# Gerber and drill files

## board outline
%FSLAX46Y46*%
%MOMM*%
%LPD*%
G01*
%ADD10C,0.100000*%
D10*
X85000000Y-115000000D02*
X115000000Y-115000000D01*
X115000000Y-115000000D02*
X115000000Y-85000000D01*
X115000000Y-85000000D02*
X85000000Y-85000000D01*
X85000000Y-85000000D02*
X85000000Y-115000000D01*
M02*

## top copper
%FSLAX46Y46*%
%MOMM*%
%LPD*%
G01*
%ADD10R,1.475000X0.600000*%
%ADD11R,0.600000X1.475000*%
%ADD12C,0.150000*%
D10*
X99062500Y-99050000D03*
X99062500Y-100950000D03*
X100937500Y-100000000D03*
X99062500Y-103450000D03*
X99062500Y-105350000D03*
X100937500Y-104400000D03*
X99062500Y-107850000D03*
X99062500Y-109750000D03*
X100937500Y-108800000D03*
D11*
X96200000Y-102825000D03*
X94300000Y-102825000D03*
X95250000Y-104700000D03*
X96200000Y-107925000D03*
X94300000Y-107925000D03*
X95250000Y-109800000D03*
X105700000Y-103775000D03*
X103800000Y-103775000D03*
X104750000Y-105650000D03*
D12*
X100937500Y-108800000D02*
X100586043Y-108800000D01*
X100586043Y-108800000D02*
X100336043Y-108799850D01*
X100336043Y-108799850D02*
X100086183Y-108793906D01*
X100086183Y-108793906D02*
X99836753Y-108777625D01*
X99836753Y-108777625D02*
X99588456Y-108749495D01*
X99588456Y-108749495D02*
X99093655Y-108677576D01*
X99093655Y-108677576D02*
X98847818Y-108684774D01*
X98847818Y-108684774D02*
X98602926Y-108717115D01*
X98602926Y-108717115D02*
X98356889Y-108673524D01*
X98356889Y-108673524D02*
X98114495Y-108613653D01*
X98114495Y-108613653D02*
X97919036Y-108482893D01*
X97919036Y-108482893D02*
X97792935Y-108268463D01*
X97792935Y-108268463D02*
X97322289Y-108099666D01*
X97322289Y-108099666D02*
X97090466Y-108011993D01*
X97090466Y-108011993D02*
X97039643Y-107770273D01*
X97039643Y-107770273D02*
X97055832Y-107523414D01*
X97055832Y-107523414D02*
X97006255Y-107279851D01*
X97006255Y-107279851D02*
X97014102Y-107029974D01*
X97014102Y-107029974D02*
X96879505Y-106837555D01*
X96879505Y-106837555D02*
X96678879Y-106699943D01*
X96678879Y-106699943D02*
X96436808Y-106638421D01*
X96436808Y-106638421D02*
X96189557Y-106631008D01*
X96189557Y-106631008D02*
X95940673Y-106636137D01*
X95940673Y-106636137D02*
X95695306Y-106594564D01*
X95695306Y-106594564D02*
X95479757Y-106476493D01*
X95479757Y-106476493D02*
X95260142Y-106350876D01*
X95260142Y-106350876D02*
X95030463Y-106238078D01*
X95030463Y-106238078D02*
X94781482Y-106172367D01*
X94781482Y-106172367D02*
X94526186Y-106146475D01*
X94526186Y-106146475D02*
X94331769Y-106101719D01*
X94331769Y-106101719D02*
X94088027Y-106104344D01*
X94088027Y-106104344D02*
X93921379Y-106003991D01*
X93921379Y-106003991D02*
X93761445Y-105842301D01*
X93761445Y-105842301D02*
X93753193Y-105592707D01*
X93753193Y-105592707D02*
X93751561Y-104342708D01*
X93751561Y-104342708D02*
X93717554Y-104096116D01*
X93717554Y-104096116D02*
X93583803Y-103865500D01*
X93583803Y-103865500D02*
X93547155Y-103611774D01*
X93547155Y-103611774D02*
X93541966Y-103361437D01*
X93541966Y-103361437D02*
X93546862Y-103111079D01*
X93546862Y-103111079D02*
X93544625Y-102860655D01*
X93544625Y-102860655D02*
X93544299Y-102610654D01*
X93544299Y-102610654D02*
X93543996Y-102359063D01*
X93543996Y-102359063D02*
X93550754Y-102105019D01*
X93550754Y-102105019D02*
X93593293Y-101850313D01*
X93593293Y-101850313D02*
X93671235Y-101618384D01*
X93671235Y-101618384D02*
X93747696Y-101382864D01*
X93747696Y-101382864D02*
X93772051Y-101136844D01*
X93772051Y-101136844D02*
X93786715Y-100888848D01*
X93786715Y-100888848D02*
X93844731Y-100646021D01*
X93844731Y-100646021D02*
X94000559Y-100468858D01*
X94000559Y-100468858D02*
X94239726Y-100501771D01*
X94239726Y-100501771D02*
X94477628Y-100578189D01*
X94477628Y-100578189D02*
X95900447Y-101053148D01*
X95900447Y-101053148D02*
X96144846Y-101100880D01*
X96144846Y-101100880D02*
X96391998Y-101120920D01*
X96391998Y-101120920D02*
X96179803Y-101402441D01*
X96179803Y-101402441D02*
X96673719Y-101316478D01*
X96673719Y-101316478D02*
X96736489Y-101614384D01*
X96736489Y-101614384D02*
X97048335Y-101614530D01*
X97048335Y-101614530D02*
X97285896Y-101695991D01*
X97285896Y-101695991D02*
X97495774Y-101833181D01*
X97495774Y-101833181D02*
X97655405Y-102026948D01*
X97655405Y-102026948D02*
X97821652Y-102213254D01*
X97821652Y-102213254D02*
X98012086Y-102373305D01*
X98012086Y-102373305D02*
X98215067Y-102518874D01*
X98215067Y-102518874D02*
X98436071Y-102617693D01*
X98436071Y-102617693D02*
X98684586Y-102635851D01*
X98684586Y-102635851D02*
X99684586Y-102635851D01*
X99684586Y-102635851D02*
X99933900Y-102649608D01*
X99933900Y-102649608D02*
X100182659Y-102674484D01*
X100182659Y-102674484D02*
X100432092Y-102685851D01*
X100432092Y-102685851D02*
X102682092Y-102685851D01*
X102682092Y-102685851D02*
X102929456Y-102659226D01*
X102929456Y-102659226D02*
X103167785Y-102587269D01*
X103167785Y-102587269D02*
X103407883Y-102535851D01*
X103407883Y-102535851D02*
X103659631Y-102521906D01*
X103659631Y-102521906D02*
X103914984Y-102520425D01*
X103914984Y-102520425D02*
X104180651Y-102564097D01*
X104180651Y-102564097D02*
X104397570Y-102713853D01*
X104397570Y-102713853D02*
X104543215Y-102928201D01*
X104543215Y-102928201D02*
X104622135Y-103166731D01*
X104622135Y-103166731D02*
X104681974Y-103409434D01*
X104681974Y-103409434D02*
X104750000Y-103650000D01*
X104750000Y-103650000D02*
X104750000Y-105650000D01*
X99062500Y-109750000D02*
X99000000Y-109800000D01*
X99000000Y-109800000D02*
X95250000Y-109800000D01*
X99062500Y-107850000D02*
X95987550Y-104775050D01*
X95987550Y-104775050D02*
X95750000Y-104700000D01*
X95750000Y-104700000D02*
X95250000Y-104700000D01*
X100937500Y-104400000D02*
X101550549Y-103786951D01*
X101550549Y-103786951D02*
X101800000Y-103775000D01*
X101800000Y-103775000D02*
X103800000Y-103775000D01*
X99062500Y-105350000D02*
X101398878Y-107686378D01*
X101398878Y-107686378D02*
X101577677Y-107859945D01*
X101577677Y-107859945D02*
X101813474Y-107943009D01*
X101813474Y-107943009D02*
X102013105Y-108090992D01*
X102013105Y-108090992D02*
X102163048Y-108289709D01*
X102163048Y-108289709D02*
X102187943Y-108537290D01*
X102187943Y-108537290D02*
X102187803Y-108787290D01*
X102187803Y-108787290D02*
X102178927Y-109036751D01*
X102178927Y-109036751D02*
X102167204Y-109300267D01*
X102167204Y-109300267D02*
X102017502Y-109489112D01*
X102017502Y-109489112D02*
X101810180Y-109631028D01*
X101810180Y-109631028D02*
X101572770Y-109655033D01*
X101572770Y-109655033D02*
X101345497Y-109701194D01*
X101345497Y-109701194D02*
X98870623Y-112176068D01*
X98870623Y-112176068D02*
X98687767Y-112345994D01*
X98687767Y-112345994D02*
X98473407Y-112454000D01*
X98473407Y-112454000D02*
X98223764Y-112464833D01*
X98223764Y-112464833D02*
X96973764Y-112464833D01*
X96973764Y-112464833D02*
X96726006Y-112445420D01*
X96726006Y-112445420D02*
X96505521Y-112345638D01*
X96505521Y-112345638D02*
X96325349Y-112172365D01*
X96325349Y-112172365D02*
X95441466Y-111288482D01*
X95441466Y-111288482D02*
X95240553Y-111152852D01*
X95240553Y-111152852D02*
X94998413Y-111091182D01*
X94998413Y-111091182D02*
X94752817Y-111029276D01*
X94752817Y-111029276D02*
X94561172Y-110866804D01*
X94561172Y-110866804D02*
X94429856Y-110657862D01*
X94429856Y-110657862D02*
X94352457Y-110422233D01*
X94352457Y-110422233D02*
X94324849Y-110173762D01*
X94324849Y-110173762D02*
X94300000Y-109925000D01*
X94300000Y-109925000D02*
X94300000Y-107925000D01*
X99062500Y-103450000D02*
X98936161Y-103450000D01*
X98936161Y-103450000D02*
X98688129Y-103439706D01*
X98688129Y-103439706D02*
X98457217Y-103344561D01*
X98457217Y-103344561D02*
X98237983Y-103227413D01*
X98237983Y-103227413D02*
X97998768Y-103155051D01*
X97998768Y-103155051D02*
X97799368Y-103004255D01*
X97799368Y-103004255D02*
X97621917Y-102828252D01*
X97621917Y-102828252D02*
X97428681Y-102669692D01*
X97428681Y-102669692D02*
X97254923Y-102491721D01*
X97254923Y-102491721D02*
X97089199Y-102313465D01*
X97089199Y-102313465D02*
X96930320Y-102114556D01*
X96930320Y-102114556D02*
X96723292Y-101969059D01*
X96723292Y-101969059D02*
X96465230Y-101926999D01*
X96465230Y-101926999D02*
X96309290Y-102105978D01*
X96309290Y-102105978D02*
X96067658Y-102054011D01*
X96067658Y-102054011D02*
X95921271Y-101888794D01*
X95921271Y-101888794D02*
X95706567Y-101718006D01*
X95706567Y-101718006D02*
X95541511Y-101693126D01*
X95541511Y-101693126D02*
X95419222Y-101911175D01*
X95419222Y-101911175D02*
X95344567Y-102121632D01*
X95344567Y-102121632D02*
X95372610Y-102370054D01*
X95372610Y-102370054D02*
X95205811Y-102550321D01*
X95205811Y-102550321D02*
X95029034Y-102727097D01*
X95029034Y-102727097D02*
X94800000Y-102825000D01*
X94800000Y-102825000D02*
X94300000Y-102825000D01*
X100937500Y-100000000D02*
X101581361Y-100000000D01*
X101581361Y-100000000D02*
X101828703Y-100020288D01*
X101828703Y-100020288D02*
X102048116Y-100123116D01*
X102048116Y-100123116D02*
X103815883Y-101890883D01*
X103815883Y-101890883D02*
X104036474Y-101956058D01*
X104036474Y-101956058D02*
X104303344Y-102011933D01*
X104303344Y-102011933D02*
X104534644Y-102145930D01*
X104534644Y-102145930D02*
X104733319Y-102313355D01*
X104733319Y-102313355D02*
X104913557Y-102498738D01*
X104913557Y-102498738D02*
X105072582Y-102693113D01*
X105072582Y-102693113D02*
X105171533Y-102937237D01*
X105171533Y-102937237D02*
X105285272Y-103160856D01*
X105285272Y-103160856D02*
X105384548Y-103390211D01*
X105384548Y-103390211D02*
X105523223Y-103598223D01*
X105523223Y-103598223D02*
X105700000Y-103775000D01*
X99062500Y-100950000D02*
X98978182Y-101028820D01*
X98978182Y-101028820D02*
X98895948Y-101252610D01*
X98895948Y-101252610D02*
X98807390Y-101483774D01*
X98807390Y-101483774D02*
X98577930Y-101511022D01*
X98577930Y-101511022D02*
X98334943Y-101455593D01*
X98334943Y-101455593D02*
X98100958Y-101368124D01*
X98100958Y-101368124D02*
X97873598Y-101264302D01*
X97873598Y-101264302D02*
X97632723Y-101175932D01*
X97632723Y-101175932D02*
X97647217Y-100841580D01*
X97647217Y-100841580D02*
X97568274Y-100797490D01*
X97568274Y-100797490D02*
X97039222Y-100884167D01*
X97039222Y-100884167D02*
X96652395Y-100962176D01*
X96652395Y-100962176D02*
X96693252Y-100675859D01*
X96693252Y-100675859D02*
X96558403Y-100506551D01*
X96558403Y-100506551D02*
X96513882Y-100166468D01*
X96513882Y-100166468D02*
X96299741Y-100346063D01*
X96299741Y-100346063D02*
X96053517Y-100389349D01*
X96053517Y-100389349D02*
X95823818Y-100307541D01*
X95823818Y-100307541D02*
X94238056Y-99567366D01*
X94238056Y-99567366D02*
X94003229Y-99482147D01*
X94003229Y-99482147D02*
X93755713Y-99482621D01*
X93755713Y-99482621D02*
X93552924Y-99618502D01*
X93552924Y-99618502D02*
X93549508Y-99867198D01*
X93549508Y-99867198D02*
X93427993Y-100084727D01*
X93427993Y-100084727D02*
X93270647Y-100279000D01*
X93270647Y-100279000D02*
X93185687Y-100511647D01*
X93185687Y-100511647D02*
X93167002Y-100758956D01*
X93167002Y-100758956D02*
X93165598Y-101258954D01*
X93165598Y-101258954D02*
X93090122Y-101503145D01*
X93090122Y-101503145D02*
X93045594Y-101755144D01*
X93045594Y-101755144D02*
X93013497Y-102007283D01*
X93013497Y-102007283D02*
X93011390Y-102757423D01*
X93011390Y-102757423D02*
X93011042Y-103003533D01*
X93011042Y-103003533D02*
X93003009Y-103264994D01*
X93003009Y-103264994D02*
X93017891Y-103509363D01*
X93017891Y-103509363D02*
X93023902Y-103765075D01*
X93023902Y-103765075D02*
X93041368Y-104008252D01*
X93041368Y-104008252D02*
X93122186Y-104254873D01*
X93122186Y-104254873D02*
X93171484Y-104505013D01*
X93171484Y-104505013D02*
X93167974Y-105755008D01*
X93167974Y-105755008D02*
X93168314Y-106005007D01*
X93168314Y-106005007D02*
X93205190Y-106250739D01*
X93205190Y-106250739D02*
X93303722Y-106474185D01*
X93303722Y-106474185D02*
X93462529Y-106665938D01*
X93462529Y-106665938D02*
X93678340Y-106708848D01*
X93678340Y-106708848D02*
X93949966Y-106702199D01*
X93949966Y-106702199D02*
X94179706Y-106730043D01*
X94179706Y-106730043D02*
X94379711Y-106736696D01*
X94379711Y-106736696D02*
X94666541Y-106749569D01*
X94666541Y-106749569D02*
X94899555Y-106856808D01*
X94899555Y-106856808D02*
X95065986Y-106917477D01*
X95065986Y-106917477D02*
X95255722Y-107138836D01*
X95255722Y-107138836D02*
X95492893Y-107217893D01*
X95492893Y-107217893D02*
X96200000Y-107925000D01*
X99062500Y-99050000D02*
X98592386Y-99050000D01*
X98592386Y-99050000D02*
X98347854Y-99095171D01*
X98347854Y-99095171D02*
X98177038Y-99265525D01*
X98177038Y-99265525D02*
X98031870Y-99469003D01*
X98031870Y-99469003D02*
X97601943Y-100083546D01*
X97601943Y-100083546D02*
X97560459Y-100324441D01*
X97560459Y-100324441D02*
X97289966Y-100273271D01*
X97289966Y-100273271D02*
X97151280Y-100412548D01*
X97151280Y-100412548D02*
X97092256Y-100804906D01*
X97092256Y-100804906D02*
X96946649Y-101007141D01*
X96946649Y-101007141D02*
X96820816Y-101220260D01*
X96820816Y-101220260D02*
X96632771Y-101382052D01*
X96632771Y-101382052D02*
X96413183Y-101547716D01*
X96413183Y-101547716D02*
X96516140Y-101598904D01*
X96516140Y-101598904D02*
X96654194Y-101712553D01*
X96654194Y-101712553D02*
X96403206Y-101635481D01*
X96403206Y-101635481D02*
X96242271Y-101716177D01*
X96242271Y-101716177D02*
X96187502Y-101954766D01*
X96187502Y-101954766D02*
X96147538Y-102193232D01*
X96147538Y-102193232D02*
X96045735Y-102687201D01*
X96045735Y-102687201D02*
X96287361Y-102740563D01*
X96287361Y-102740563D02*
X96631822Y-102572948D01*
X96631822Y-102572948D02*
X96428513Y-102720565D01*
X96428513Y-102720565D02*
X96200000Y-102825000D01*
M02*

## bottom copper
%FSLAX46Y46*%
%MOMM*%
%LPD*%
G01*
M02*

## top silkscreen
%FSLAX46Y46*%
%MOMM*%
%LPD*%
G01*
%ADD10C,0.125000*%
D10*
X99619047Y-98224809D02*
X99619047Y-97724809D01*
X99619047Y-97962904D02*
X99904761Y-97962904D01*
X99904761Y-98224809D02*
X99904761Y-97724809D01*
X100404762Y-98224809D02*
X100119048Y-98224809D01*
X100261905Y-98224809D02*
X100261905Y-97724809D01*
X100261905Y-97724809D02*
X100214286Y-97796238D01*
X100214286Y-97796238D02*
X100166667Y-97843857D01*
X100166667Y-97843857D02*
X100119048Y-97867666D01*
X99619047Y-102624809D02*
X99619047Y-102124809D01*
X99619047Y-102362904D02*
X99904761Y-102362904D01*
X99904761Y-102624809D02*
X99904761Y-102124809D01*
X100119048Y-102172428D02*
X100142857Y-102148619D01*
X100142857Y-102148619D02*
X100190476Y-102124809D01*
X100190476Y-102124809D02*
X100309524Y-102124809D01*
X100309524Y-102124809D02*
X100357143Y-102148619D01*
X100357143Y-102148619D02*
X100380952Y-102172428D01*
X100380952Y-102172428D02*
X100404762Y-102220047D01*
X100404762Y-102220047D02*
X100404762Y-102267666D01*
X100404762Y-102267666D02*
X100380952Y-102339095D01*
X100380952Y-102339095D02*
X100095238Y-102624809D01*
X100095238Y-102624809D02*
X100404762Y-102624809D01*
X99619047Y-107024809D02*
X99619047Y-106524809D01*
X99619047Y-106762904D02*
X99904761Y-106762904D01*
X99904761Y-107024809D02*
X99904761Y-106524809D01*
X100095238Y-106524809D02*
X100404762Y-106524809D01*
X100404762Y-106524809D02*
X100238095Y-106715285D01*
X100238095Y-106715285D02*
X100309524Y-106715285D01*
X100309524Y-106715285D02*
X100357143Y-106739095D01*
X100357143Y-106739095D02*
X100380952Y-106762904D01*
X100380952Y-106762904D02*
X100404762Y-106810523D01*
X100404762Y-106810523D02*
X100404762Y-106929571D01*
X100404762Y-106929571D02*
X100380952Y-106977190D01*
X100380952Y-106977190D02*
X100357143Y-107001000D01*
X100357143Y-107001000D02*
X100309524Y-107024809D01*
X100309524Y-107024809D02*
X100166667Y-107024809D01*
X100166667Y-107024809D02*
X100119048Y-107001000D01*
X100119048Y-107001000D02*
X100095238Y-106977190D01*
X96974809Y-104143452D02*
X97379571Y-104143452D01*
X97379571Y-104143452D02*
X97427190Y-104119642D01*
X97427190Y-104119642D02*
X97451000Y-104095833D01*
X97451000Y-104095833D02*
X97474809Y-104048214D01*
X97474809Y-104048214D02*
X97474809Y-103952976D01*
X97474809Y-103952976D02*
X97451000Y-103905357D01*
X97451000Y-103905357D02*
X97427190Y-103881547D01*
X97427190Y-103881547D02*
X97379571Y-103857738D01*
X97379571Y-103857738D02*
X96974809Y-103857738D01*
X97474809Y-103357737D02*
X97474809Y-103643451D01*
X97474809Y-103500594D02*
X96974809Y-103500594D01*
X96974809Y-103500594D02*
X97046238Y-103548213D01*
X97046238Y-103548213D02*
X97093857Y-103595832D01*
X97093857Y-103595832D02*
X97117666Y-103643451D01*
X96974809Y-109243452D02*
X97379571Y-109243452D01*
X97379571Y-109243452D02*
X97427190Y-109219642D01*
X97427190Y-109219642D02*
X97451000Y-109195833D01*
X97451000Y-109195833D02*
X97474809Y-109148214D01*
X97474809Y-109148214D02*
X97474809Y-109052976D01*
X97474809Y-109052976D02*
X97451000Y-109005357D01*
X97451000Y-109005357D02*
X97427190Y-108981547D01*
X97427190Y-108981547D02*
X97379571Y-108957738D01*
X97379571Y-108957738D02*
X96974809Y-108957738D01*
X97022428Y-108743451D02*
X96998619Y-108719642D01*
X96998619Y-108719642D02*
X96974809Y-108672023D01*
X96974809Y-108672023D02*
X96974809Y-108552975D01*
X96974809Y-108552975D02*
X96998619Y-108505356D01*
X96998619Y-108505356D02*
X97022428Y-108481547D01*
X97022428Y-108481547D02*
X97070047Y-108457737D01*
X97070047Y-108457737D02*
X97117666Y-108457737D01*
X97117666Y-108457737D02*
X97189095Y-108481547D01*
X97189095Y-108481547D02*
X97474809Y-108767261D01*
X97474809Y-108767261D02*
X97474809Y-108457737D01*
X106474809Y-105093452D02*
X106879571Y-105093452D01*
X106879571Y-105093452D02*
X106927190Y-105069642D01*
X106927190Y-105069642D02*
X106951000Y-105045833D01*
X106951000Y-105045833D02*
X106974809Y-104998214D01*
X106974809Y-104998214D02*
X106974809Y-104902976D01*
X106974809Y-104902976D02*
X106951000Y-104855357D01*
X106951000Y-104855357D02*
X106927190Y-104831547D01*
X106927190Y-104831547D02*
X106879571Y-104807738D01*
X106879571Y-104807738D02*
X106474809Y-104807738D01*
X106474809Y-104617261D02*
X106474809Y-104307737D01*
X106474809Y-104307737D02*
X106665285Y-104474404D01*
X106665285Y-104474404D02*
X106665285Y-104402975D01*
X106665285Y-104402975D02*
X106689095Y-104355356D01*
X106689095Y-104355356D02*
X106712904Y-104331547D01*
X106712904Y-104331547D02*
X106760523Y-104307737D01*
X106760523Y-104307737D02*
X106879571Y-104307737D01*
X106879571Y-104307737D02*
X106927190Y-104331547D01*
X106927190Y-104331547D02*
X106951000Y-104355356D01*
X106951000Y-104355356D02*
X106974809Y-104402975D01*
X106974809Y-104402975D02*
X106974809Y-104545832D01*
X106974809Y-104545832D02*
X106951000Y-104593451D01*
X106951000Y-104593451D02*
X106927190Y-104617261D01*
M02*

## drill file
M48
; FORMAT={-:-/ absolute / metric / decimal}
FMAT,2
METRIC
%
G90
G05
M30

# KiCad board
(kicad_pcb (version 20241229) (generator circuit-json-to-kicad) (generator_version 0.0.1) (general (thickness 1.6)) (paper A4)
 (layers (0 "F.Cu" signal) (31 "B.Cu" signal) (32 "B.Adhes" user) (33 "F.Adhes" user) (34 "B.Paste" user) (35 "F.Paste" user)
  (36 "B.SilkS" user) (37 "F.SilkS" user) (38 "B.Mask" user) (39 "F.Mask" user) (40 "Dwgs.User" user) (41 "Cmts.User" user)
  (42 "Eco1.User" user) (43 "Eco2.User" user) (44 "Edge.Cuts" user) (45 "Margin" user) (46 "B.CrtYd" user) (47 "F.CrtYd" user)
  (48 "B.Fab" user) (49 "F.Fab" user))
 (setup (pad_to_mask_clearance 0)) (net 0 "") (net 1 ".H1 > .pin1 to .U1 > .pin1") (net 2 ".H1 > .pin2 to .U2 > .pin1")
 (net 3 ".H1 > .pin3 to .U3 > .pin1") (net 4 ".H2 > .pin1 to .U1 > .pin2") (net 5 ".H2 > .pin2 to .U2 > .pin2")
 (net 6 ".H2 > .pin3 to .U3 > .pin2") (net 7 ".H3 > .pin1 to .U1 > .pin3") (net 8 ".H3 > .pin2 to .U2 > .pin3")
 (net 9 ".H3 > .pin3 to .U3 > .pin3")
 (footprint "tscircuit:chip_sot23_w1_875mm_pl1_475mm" (layer F.Cu) (at 100 100 0)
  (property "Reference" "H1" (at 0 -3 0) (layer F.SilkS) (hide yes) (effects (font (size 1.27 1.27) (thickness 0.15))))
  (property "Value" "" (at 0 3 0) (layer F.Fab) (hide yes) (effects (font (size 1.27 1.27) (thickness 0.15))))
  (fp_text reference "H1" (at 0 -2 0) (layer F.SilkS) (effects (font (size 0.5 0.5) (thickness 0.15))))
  (pad "1" smd rect (at -0.9375 -0.95 0) (size 1.475 0.6) (layers F.Cu F.Mask) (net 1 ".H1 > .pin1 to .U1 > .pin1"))
  (pad "2" smd rect (at -0.9375 0.95 0) (size 1.475 0.6) (layers F.Cu F.Mask) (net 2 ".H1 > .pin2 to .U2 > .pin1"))
  (pad "3" smd rect (at 0.9375 0 0) (size 1.475 0.6) (layers F.Cu F.Mask) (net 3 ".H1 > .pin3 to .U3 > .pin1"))
  (pad "" smd rect (at -0.9375 -0.95 0) (size 1.0325 0.42) (layers F.Paste))
  (pad "" smd rect (at -0.9375 0.95 0) (size 1.0325 0.42) (layers F.Paste))
  (pad "" smd rect (at 0.9375 0 0) (size 1.0325 0.42) (layers F.Paste)))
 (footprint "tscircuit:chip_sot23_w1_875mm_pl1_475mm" (layer F.Cu) (at 100 104.4 0)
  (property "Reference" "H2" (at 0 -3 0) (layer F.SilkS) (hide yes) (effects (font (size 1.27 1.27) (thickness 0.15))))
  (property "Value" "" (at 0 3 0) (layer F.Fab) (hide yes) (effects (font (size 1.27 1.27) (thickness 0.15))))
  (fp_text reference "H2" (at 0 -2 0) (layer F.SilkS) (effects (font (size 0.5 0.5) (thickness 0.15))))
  (pad "1" smd rect (at -0.9375 -0.9500000000000002 0) (size 1.475 0.6) (layers F.Cu F.Mask) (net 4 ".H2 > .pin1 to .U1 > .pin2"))
  (pad "2" smd rect (at -0.9375 0.9500000000000002 0) (size 1.475 0.6) (layers F.Cu F.Mask) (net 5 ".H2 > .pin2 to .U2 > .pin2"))
  (pad "3" smd rect (at 0.9375 0 0) (size 1.475 0.6) (layers F.Cu F.Mask) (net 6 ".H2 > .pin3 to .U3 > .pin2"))
  (pad "" smd rect (at -0.9375 -0.9500000000000002 0) (size 1.0325 0.42) (layers F.Paste))
  (pad "" smd rect (at -0.9375 0.9500000000000002 0) (size 1.0325 0.42) (layers F.Paste))
  (pad "" smd rect (at 0.9375 0 0) (size 1.0325 0.42) (layers F.Paste)))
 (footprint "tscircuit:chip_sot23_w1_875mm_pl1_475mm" (layer F.Cu) (at 100 108.8 0)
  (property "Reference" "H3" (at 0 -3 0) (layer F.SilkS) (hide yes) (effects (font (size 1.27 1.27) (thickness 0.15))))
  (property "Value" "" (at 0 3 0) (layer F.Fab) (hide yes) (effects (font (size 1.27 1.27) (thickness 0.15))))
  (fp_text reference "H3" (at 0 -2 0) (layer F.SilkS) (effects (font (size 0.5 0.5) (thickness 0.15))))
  (pad "1" smd rect (at -0.9375 -0.9500000000000002 0) (size 1.475 0.6) (layers F.Cu F.Mask) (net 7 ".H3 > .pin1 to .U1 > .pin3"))
  (pad "2" smd rect (at -0.9375 0.9499999999999993 0) (size 1.475 0.6) (layers F.Cu F.Mask) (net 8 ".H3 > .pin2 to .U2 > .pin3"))
  (pad "3" smd rect (at 0.9375 0 0) (size 1.475 0.6) (layers F.Cu F.Mask) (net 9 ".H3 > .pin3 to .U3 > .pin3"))
  (pad "" smd rect (at -0.9375 -0.9500000000000002 0) (size 1.0325 0.42) (layers F.Paste))
  (pad "" smd rect (at -0.9375 0.9499999999999993 0) (size 1.0325 0.42) (layers F.Paste))
  (pad "" smd rect (at 0.9375 0 0) (size 1.0325 0.42) (layers F.Paste)))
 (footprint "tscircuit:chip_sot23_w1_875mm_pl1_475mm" (layer F.Cu) (at 95.25 103.7625 -90.00000000000001)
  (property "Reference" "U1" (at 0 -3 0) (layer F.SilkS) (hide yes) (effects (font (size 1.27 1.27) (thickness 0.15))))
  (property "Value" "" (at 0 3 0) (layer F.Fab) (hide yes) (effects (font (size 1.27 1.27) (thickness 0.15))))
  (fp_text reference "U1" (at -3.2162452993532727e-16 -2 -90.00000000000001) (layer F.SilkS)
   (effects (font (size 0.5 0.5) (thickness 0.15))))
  (pad "1" smd rect (at -0.9375000000000004 -0.9499999999999993 0) (size 0.6 1.475) (layers F.Cu F.Mask)
   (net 1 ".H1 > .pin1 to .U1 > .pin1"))
  (pad "2" smd rect (at -0.9374999999999996 0.9500000000000011 0) (size 0.6 1.475) (layers F.Cu F.Mask) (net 4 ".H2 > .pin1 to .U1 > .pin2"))
  (pad "3" smd rect (at 0.9375 0 0) (size 0.6 1.475) (layers F.Cu F.Mask) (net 7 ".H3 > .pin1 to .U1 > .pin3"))
  (pad "" smd rect (at -0.9375000000000004 -0.9499999999999993 0) (size 0.42 1.0325) (layers F.Paste))
  (pad "" smd rect (at -0.9374999999999996 0.9500000000000011 0) (size 0.42 1.0325) (layers F.Paste))
  (pad "" smd rect (at 0.9375 0 0) (size 0.42 1.0325) (layers F.Paste)))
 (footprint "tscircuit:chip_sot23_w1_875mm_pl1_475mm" (layer F.Cu) (at 95.25 108.8625 -90.00000000000001)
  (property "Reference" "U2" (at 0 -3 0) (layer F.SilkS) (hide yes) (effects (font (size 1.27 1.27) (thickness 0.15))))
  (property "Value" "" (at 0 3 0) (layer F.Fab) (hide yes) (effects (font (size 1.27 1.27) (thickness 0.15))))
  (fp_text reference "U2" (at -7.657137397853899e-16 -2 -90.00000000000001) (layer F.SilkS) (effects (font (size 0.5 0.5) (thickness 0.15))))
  (pad "1" smd rect (at -0.9375 -0.9499999999999997 0) (size 0.6 1.475) (layers F.Cu F.Mask) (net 2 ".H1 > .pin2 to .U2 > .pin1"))
  (pad "2" smd rect (at -0.9375 0.9500000000000011 0) (size 0.6 1.475) (layers F.Cu F.Mask) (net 5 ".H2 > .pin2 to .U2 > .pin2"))
  (pad "3" smd rect (at 0.9375 0 0) (size 0.6 1.475) (layers F.Cu F.Mask) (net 8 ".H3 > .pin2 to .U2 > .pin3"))
  (pad "" smd rect (at -0.9375 -0.9499999999999997 0) (size 0.42 1.0325) (layers F.Paste))
  (pad "" smd rect (at -0.9375 0.9500000000000011 0) (size 0.42 1.0325) (layers F.Paste))
  (pad "" smd rect (at 0.9375 0 0) (size 0.42 1.0325) (layers F.Paste)))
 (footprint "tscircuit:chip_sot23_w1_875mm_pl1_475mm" (layer F.Cu) (at 104.75 104.7125 -90.00000000000001)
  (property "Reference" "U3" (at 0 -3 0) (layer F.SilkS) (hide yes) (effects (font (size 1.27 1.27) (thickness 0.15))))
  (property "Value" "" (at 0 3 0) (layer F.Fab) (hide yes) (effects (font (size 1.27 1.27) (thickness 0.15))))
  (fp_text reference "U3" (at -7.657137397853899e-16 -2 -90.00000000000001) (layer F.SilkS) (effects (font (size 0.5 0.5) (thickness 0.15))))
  (pad "1" smd rect (at -0.9375000000000004 -0.9500000000000002 0) (size 0.6 1.475) (layers F.Cu F.Mask)
   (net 3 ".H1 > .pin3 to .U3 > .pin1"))
  (pad "2" smd rect (at -0.9374999999999996 0.9500000000000002 0) (size 0.6 1.475) (layers F.Cu F.Mask) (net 6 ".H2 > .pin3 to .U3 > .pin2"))
  (pad "3" smd rect (at 0.9375 0 0) (size 0.6 1.475) (layers F.Cu F.Mask) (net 9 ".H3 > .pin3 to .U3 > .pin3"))
  (pad "" smd rect (at -0.9375000000000004 -0.9500000000000002 0) (size 0.42 1.0325) (layers F.Paste))
  (pad "" smd rect (at -0.9374999999999996 0.9500000000000002 0) (size 0.42 1.0325) (layers F.Paste))
  (pad "" smd rect (at 0.9375 0 0) (size 0.42 1.0325) (layers F.Paste)))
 (segment (start 100.9375 108.8) (end 100.58604316307064 108.8) (width 0.15) (layer F.Cu) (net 9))
 (segment (start 100.58604316307064 108.8) (end 100.33604325630263 108.79985032467384) (width 0.15) (layer F.Cu) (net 9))
 (segment (start 100.33604325630263 108.79985032467384) (end 100.086182582394 108.7939062426908) (width 0.15) (layer F.Cu) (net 9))
 (segment (start 100.086182582394 108.7939062426908) (end 99.83675258768096 108.77762494052355) (width 0.15) (layer F.Cu) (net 9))
 (segment (start 99.83675258768096 108.77762494052355) (end 99.5884561425144 108.74949464263153) (width 0.15) (layer F.Cu) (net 9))
 (segment (start 99.5884561425144 108.74949464263153) (end 99.09365546986794 108.6775759778177) (width 0.15) (layer F.Cu) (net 9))
 (segment (start 99.09365546986794 108.6775759778177) (end 98.84781760378522 108.68477395432264) (width 0.15) (layer F.Cu) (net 9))
 (segment (start 98.84781760378522 108.68477395432264) (end 98.6029257798537 108.71711459527816) (width 0.15) (layer F.Cu) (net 9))
 (segment (start 98.6029257798537 108.71711459527816) (end 98.35688941387995 108.6735236468046) (width 0.15) (layer F.Cu) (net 9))
 (segment (start 98.35688941387995 108.6735236468046) (end 98.1144951003154 108.61365317525244) (width 0.15) (layer F.Cu) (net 9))
 (segment (start 98.1144951003154 108.61365317525244) (end 97.91903634515725 108.48289257852745) (width 0.15) (layer F.Cu) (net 9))
 (segment (start 97.91903634515725 108.48289257852745) (end 97.79293472388505 108.26846256762974) (width 0.15) (layer F.Cu) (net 9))
 (segment (start 97.79293472388505 108.26846256762974) (end 97.3222887689124 108.09966569245758) (width 0.15) (layer F.Cu) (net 9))
 (segment (start 97.3222887689124 108.09966569245758) (end 97.0904659355959 108.01199297313701) (width 0.15) (layer F.Cu) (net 9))
 (segment (start 97.0904659355959 108.01199297313701) (end 97.03964293065343 107.77027276830762) (width 0.15) (layer F.Cu) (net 9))
 (segment (start 97.03964293065343 107.77027276830762) (end 97.05583182611103 107.52341402424582) (width 0.15) (layer F.Cu) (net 9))
 (segment (start 97.05583182611103 107.52341402424582) (end 97.0062547177474 107.27985068013375) (width 0.15) (layer F.Cu) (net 9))
 (segment (start 97.0062547177474 107.27985068013375) (end 97.0141018447695 107.02997386528791) (width 0.15) (layer F.Cu) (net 9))
 (segment (start 97.0141018447695 107.02997386528791) (end 96.87950485613383 106.83755522887635) (width 0.15) (layer F.Cu) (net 9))
 (segment (start 96.87950485613383 106.83755522887635) (end 96.67887900732497 106.69994305064326) (width 0.15) (layer F.Cu) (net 9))
 (segment (start 96.67887900732497 106.69994305064326) (end 96.43680768799454 106.63842130728048) (width 0.15) (layer F.Cu) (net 9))
 (segment (start 96.43680768799454 106.63842130728048) (end 96.18955667286622 106.63100802970678) (width 0.15) (layer F.Cu) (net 9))
 (segment (start 96.18955667286622 106.63100802970678) (end 95.94067347881345 106.63613720101705) (width 0.15) (layer F.Cu) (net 9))
 (segment (start 95.94067347881345 106.63613720101705) (end 95.69530620165742 106.59456392455309) (width 0.15) (layer F.Cu) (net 9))
 (segment (start 95.69530620165742 106.59456392455309) (end 95.47975677696712 106.47649346616738) (width 0.15) (layer F.Cu) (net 9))
 (segment (start 95.47975677696712 106.47649346616738) (end 95.2601422924707 106.35087587239283) (width 0.15) (layer F.Cu) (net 9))
 (segment (start 95.2601422924707 106.35087587239283) (end 95.03046341175923 106.23807812989479) (width 0.15) (layer F.Cu) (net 9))
 (segment (start 95.03046341175923 106.23807812989479) (end 94.78148248959153 106.17236733531573) (width 0.15) (layer F.Cu) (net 9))
 (segment (start 94.78148248959153 106.17236733531573) (end 94.52618636298615 106.14647525815256) (width 0.15) (layer F.Cu) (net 9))
 (segment (start 94.52618636298615 106.14647525815256) (end 94.33176907888343 106.10171923993316) (width 0.15) (layer F.Cu) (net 9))
 (segment (start 94.33176907888343 106.10171923993316) (end 94.08802719542254 106.10434396112815) (width 0.15) (layer F.Cu) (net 9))
 (segment (start 94.08802719542254 106.10434396112815) (end 93.9213792736493 106.00399076505865) (width 0.15) (layer F.Cu) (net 9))
 (segment (start 93.9213792736493 106.00399076505865) (end 93.76144489605181 105.84230109615851) (width 0.15) (layer F.Cu) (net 9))
 (segment (start 93.76144489605181 105.84230109615851) (end 93.75319274666023 105.59270698479696) (width 0.15) (layer F.Cu) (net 9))
 (segment (start 93.75319274666023 105.59270698479696) (end 93.75156063799724 104.3427080503089) (width 0.15) (layer F.Cu) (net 9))
 (segment (start 93.75156063799724 104.3427080503089) (end 93.71755416731226 104.09611593614386) (width 0.15) (layer F.Cu) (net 9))
 (segment (start 93.71755416731226 104.09611593614386) (end 93.58380321069716 103.86549957100326) (width 0.15) (layer F.Cu) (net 9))
 (segment (start 93.58380321069716 103.86549957100326) (end 93.54715505014157 103.61177377060514) (width 0.15) (layer F.Cu) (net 9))
 (segment (start 93.54715505014157 103.61177377060514) (end 93.54196556639758 103.36143735779976) (width 0.15) (layer F.Cu) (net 9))
 (segment (start 93.54196556639758 103.36143735779976) (end 93.54686226794024 103.11107865438251) (width 0.15) (layer F.Cu) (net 9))
 (segment (start 93.54686226794024 103.11107865438251) (end 93.54462536441818 102.86065508614242) (width 0.15) (layer F.Cu) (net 9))
 (segment (start 93.54462536441818 102.86065508614242) (end 93.5442989414233 102.61065432627855) (width 0.15) (layer F.Cu) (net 9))
 (segment (start 93.5442989414233 102.61065432627855) (end 93.54399635791543 102.35906279706859) (width 0.15) (layer F.Cu) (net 9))
 (segment (start 93.54399635791543 102.35906279706859) (end 93.55075416462132 102.10501853637236) (width 0.15) (layer F.Cu) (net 9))
 (segment (start 93.55075416462132 102.10501853637236) (end 93.59329273959793 101.85031254374815) (width 0.15) (layer F.Cu) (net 9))
 (segment (start 93.59329273959793 101.85031254374815) (end 93.67123541734576 101.61838405567444) (width 0.15) (layer F.Cu) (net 9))
 (segment (start 93.67123541734576 101.61838405567444) (end 93.74769600451228 101.38286361841507) (width 0.15) (layer F.Cu) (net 9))
 (segment (start 93.74769600451228 101.38286361841507) (end 93.77205079353223 101.1368435093673) (width 0.15) (layer F.Cu) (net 9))
 (segment (start 93.77205079353223 101.1368435093673) (end 93.78671545473954 100.8888481612233) (width 0.15) (layer F.Cu) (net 9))
 (segment (start 93.78671545473954 100.8888481612233) (end 93.84473089290482 100.64602146131554) (width 0.15) (layer F.Cu) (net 9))
 (segment (start 93.84473089290482 100.64602146131554) (end 94.00055935074698 100.46885765388244) (width 0.15) (layer F.Cu) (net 9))
 (segment (start 94.00055935074698 100.46885765388244) (end 94.23972594047453 100.50177064336572) (width 0.15) (layer F.Cu) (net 9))
 (segment (start 94.23972594047453 100.50177064336572) (end 94.47762800052683 100.57818940480014) (width 0.15) (layer F.Cu) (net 9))
 (segment (start 94.47762800052683 100.57818940480014) (end 95.90044720420468 101.0531478383978) (width 0.15) (layer F.Cu) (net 9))
 (segment (start 95.90044720420468 101.0531478383978) (end 96.14484595532093 101.1008795328863) (width 0.15) (layer F.Cu) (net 9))
 (segment (start 96.14484595532093 101.1008795328863) (end 96.39199847027233 101.12092018490358) (width 0.15) (layer F.Cu) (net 9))
 (segment (start 96.39199847027233 101.12092018490358) (end 96.17980291806218 101.40244075589425) (width 0.15) (layer F.Cu) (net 9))
 (segment (start 96.17980291806218 101.40244075589425) (end 96.67371867500096 101.31647795920247) (width 0.15) (layer F.Cu) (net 9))
 (segment (start 96.67371867500096 101.31647795920247) (end 96.73648880734723 101.61438428635626) (width 0.15) (layer F.Cu) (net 9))
 (segment (start 96.73648880734723 101.61438428635626) (end 97.04833485790812 101.61453025161605) (width 0.15) (layer F.Cu) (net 9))
 (segment (start 97.04833485790812 101.61453025161605) (end 97.28589646973133 101.6959906429369) (width 0.15) (layer F.Cu) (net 9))
 (segment (start 97.28589646973133 101.6959906429369) (end 97.4957735906842 101.83318066540177) (width 0.15) (layer F.Cu) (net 9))
 (segment (start 97.4957735906842 101.83318066540177) (end 97.65540487592243 102.026947921416) (width 0.15) (layer F.Cu) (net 9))
 (segment (start 97.65540487592243 102.026947921416) (end 97.82165191792967 102.2132538219729) (width 0.15) (layer F.Cu) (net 9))
 (segment (start 97.82165191792967 102.2132538219729) (end 98.01208618634267 102.3733045437575) (width 0.15) (layer F.Cu) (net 9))
 (segment (start 98.01208618634267 102.3733045437575) (end 98.21506686176619 102.51887415109142) (width 0.15) (layer F.Cu) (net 9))
 (segment (start 98.21506686176619 102.51887415109142) (end 98.43607132132885 102.61769270853428) (width 0.15) (layer F.Cu) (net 9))
 (segment (start 98.43607132132885 102.61769270853428) (end 98.68458605084086 102.63585132779501) (width 0.15) (layer F.Cu) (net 9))
 (segment (start 98.68458605084086 102.63585132779501) (end 99.68458605084086 102.63585132779501) (width 0.15) (layer F.Cu) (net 9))
 (segment (start 99.68458605084086 102.63585132779501) (end 99.93389991486771 102.64960826871584) (width 0.15) (layer F.Cu) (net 9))
 (segment (start 99.93389991486771 102.64960826871584) (end 100.1826592124202 102.67448419847109) (width 0.15) (layer F.Cu) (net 9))
 (segment (start 100.1826592124202 102.67448419847109) (end 100.43209226978482 102.685851327795) (width 0.15) (layer F.Cu) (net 9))
 (segment (start 100.43209226978482 102.685851327795) (end 102.68209226978482 102.685851327795) (width 0.15) (layer F.Cu) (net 9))
 (segment (start 102.68209226978482 102.685851327795) (end 102.9294558680585 102.65922625531518) (width 0.15) (layer F.Cu) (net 9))
 (segment (start 102.9294558680585 102.65922625531518) (end 103.16778527364762 102.5872694205997) (width 0.15) (layer F.Cu) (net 9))
 (segment (start 103.16778527364762 102.5872694205997) (end 103.40788305374845 102.53585132779502) (width 0.15) (layer F.Cu) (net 9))
 (segment (start 103.40788305374845 102.53585132779502) (end 103.65963053165791 102.52190625495642) (width 0.15) (layer F.Cu) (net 9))
 (segment (start 103.65963053165791 102.52190625495642) (end 103.91498413239934 102.52042485527014) (width 0.15) (layer F.Cu) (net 9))
 (segment (start 103.91498413239934 102.52042485527014) (end 104.18065065293072 102.56409725217904) (width 0.15) (layer F.Cu) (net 9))
 (segment (start 104.18065065293072 102.56409725217904) (end 104.39757012535104 102.71385268345034) (width 0.15) (layer F.Cu) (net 9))
 (segment (start 104.39757012535104 102.71385268345034) (end 104.54321511865945 102.9282011507897) (width 0.15) (layer F.Cu) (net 9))
 (segment (start 104.54321511865945 102.9282011507897) (end 104.62213509098983 103.16673131233615) (width 0.15) (layer F.Cu) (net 9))
 (segment (start 104.62213509098983 103.16673131233615) (end 104.68197432848304 103.40943377434402) (width 0.15) (layer F.Cu) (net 9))
 (segment (start 104.68197432848304 103.40943377434402) (end 104.75 103.65) (width 0.15) (layer F.Cu) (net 9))
 (segment (start 104.75 103.65) (end 104.75 105.65) (width 0.15) (layer F.Cu) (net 9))
 (segment (start 99.0625 109.75) (end 99 109.8) (width 0.15) (layer F.Cu) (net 8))
 (segment (start 99 109.8) (end 95.25 109.8) (width 0.15) (layer F.Cu) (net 8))
 (segment (start 99.0625 107.85) (end 95.98755045166912 104.77505045166913) (width 0.15) (layer F.Cu) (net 7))
 (segment (start 95.98755045166912 104.77505045166913) (end 95.75 104.7) (width 0.15) (layer F.Cu) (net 7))
 (segment (start 95.75 104.7) (end 95.25 104.7) (width 0.15) (layer F.Cu) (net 7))
 (segment (start 100.9375 104.4) (end 101.55054876489105 103.78695123510896) (width 0.15) (layer F.Cu) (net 6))
 (segment (start 101.55054876489105 103.78695123510896) (end 101.8 103.775) (width 0.15) (layer F.Cu) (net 6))
 (segment (start 101.8 103.775) (end 103.8 103.775) (width 0.15) (layer F.Cu) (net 6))
 (segment (start 99.0625 105.35) (end 101.39887822939532 107.68637822939533) (width 0.15) (layer F.Cu) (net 5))
 (segment (start 101.39887822939532 107.68637822939533) (end 101.57767661480224 107.8599448895166) (width 0.15) (layer F.Cu) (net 5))
 (segment (start 101.57767661480224 107.8599448895166) (end 101.81347401419401 107.94300863877025) (width 0.15) (layer F.Cu) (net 5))
 (segment (start 101.81347401419401 107.94300863877025) (end 102.01310481617375 108.09099151266315) (width 0.15) (layer F.Cu) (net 5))
 (segment (start 102.01310481617375 108.09099151266315) (end 102.16304848402764 108.28970879811375) (width 0.15) (layer F.Cu) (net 5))
 (segment (start 102.16304848402764 108.28970879811375) (end 102.18794256530816 108.53729046616614) (width 0.15) (layer F.Cu) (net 5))
 (segment (start 102.18794256530816 108.53729046616614) (end 102.18780293994708 108.7872903466949) (width 0.15) (layer F.Cu) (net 5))
 (segment (start 102.18780293994708 108.7872903466949) (end 102.17892651796224 109.03675095749921) (width 0.15) (layer F.Cu) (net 5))
 (segment (start 102.17892651796224 109.03675095749921) (end 102.16720411598295 109.30026658878307) (width 0.15) (layer F.Cu) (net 5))
 (segment (start 102.16720411598295 109.30026658878307) (end 102.0175021560855 109.48911240933045) (width 0.15) (layer F.Cu) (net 5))
 (segment (start 102.0175021560855 109.48911240933045) (end 101.81017963176475 109.63102805687112) (width 0.15) (layer F.Cu) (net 5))
 (segment (start 101.81017963176475 109.63102805687112) (end 101.57277042465456 109.65503314478376) (width 0.15) (layer F.Cu) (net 5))
 (segment (start 101.57277042465456 109.65503314478376) (end 101.34549665897265 109.701193770668) (width 0.15) (layer F.Cu) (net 5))
 (segment (start 101.34549665897265 109.701193770668) (end 98.87062292481973 112.1760675048209) (width 0.15) (layer F.Cu) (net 5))
 (segment (start 98.87062292481973 112.1760675048209) (end 98.68776683720877 112.34599367301834) (width 0.15) (layer F.Cu) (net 5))
 (segment (start 98.68776683720877 112.34599367301834) (end 98.47340726824802 112.45400005753906) (width 0.15) (layer F.Cu) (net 5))
 (segment (start 98.47340726824802 112.45400005753906) (end 98.22376360134139 112.4648333349973) (width 0.15) (layer F.Cu) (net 5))
 (segment (start 98.22376360134139 112.4648333349973) (end 96.97376360134139 112.4648333349973) (width 0.15) (layer F.Cu) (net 5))
 (segment (start 96.97376360134139 112.4648333349973) (end 96.72600619435666 112.44542044961491) (width 0.15) (layer F.Cu) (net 5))
 (segment (start 96.72600619435666 112.44542044961491) (end 96.50552134432716 112.34563794153097) (width 0.15) (layer F.Cu) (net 5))
 (segment (start 96.50552134432716 112.34563794153097) (end 96.32534915708389 112.17236505434575) (width 0.15) (layer F.Cu) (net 5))
 (segment (start 96.32534915708389 112.17236505434575) (end 95.4414656806007 111.28848157786257) (width 0.15) (layer F.Cu) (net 5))
 (segment (start 95.4414656806007 111.28848157786257) (end 95.24055311317231 111.15285243405208) (width 0.15) (layer F.Cu) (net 5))
 (segment (start 95.24055311317231 111.15285243405208) (end 94.9984134737641 111.0911818908658) (width 0.15) (layer F.Cu) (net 5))
 (segment (start 94.9984134737641 111.0911818908658) (end 94.75281684399565 111.02927634345184) (width 0.15) (layer F.Cu) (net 5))
 (segment (start 94.75281684399565 111.02927634345184) (end 94.56117184451132 110.86680420992533) (width 0.15) (layer F.Cu) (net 5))
 (segment (start 94.56117184451132 110.86680420992533) (end 94.42985576902822 110.65786247998469) (width 0.15) (layer F.Cu) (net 5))
 (segment (start 94.42985576902822 110.65786247998469) (end 94.35245690279916 110.42223278659276) (width 0.15) (layer F.Cu) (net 5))
 (segment (start 94.35245690279916 110.42223278659276) (end 94.32484902128044 110.17376185292434) (width 0.15) (layer F.Cu) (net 5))
 (segment (start 94.32484902128044 110.17376185292434) (end 94.3 109.925) (width 0.15) (layer F.Cu) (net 5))
 (segment (start 94.3 109.925) (end 94.3 107.925) (width 0.15) (layer F.Cu) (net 5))
 (segment (start 99.0625 103.45) (end 98.93616054716948 103.45) (width 0.15) (layer F.Cu) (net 4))
 (segment (start 98.93616054716948 103.45) (end 98.68812913433162 103.43970610381218) (width 0.15) (layer F.Cu) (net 4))
 (segment (start 98.68812913433162 103.43970610381218) (end 98.45721747727556 103.34456138131459) (width 0.15) (layer F.Cu) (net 4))
 (segment (start 98.45721747727556 103.34456138131459) (end 98.23798292099998 103.22741263978602) (width 0.15) (layer F.Cu) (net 4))
 (segment (start 98.23798292099998 103.22741263978602) (end 97.9987684954185 103.15505125640826) (width 0.15) (layer F.Cu) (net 4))
 (segment (start 97.9987684954185 103.15505125640826) (end 97.79936789360215 103.0042553678858) (width 0.15) (layer F.Cu) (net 4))
 (segment (start 97.79936789360215 103.0042553678858) (end 97.62191735881602 102.82825249533981) (width 0.15) (layer F.Cu) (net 4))
 (segment (start 97.62191735881602 102.82825249533981) (end 97.42868142237151 102.66969219326239) (width 0.15) (layer F.Cu) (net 4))
 (segment (start 97.42868142237151 102.66969219326239) (end 97.2549233002189 102.49172109961914) (width 0.15) (layer F.Cu) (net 4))
 (segment (start 97.2549233002189 102.49172109961914) (end 97.08919927642552 102.31346498592892) (width 0.15) (layer F.Cu) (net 4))
 (segment (start 97.08919927642552 102.31346498592892) (end 96.93031959355956 102.11455562933477) (width 0.15) (layer F.Cu) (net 4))
 (segment (start 96.93031959355956 102.11455562933477) (end 96.7232921158743 101.96905884994415) (width 0.15) (layer F.Cu) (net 4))
 (segment (start 96.7232921158743 101.96905884994415) (end 96.46523048276293 101.92699934756395) (width 0.15) (layer F.Cu) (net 4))
 (segment (start 96.46523048276293 101.92699934756395) (end 96.30928962385343 102.10597814855211) (width 0.15) (layer F.Cu) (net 4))
 (segment (start 96.30928962385343 102.10597814855211) (end 96.06765771342467 102.05401140512191) (width 0.15) (layer F.Cu) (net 4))
 (segment (start 96.06765771342467 102.05401140512191) (end 95.92127102211677 101.88879425135228) (width 0.15) (layer F.Cu) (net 4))
 (segment (start 95.92127102211677 101.88879425135228) (end 95.70656717153472 101.71800640311189) (width 0.15) (layer F.Cu) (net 4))
 (segment (start 95.70656717153472 101.71800640311189) (end 95.54151118265469 101.69312643226765) (width 0.15) (layer F.Cu) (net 4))
 (segment (start 95.54151118265469 101.69312643226765) (end 95.41922192897249 101.91117536813721) (width 0.15) (layer F.Cu) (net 4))
 (segment (start 95.41922192897249 101.91117536813721) (end 95.34456741301479 102.12163184580646) (width 0.15) (layer F.Cu) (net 4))
 (segment (start 95.34456741301479 102.12163184580646) (end 95.37261043487482 102.370054044744) (width 0.15) (layer F.Cu) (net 4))
 (segment (start 95.37261043487482 102.370054044744) (end 95.20581094859259 102.55032074664102) (width 0.15) (layer F.Cu) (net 4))
 (segment (start 95.20581094859259 102.55032074664102) (end 95.02903425329595 102.72709744193766) (width 0.15) (layer F.Cu) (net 4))
 (segment (start 95.02903425329595 102.72709744193766) (end 94.8 102.825) (width 0.15) (layer F.Cu) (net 4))
 (segment (start 94.8 102.825) (end 94.3 102.825) (width 0.15) (layer F.Cu) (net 4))
 (segment (start 100.9375 100) (end 101.58136149955507 100) (width 0.15) (layer F.Cu) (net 3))
 (segment (start 101.58136149955507 100) (end 101.82870259147163 100.02028794480334) (width 0.15) (layer F.Cu) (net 3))
 (segment (start 101.82870259147163 100.02028794480334) (end 102.04811600125753 100.12311600125753) (width 0.15) (layer F.Cu) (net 3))
 (segment (start 102.04811600125753 100.12311600125753) (end 103.8158829542239 101.8908829542239) (width 0.15) (layer F.Cu) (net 3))
 (segment (start 103.8158829542239 101.8908829542239) (end 104.03647358319579 101.95605802926451) (width 0.15) (layer F.Cu) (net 3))
 (segment (start 104.03647358319579 101.95605802926451) (end 104.30334429917085 102.01193326851943) (width 0.15) (layer F.Cu) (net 3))
 (segment (start 104.30334429917085 102.01193326851943) (end 104.53464369954249 102.14593014015485) (width 0.15) (layer F.Cu) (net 3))
 (segment (start 104.53464369954249 102.14593014015485) (end 104.73331898246506 102.3133554722175) (width 0.15) (layer F.Cu) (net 3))
 (segment (start 104.73331898246506 102.3133554722175) (end 104.91355674520818 102.49873817717352) (width 0.15) (layer F.Cu) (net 3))
 (segment (start 104.91355674520818 102.49873817717352) (end 105.0725822056188 102.6931128662063) (width 0.15) (layer F.Cu) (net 3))
 (segment (start 105.0725822056188 102.6931128662063) (end 105.171532636344 102.93723659118051) (width 0.15) (layer F.Cu) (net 3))
 (segment (start 105.171532636344 102.93723659118051) (end 105.28527240868827 103.16085567753257) (width 0.15) (layer F.Cu) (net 3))
 (segment (start 105.28527240868827 103.16085567753257) (end 105.38454825564706 103.3902107311189) (width 0.15) (layer F.Cu) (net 3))
 (segment (start 105.38454825564706 103.3902107311189) (end 105.52322330470336 103.59822330470337) (width 0.15) (layer F.Cu) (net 3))
 (segment (start 105.52322330470336 103.59822330470337) (end 105.7 103.775) (width 0.15) (layer F.Cu) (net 3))
 (segment (start 99.0625 100.95) (end 98.97818221928148 101.02881989993827) (width 0.15) (layer F.Cu) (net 2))
 (segment (start 98.97818221928148 101.02881989993827) (end 98.8959478152866 101.25260977440684) (width 0.15) (layer F.Cu) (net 2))
 (segment (start 98.8959478152866 101.25260977440684) (end 98.8073903775156 101.48377368584674) (width 0.15) (layer F.Cu) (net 2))
 (segment (start 98.8073903775156 101.48377368584674) (end 98.57793043709326 101.51102246912279) (width 0.15) (layer F.Cu) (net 2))
 (segment (start 98.57793043709326 101.51102246912279) (end 98.33494300433169 101.45559264426983) (width 0.15) (layer F.Cu) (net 2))
 (segment (start 98.33494300433169 101.45559264426983) (end 98.10095804434438 101.3681240799002) (width 0.15) (layer F.Cu) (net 2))
 (segment (start 98.10095804434438 101.3681240799002) (end 97.87359839515486 101.2643024301084) (width 0.15) (layer F.Cu) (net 2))
 (segment (start 97.87359839515486 101.2643024301084) (end 97.63272324022608 101.17593191391826) (width 0.15) (layer F.Cu) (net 2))
 (segment (start 97.63272324022608 101.17593191391826) (end 97.64721707344125 100.84158020427081) (width 0.15) (layer F.Cu) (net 2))
 (segment (start 97.64721707344125 100.84158020427081) (end 97.56827390278653 100.79749007481475) (width 0.15) (layer F.Cu) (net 2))
 (segment (start 97.56827390278653 100.79749007481475) (end 97.03922177126496 100.88416748926731) (width 0.15) (layer F.Cu) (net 2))
 (segment (start 97.03922177126496 100.88416748926731) (end 96.65239517183453 100.96217647470445) (width 0.15) (layer F.Cu) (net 2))
 (segment (start 96.65239517183453 100.96217647470445) (end 96.69325183387716 100.6758585156597) (width 0.15) (layer F.Cu) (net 2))
 (segment (start 96.69325183387716 100.6758585156597) (end 96.55840266144963 100.50655060756186) (width 0.15) (layer F.Cu) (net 2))
 (segment (start 96.55840266144963 100.50655060756186) (end 96.51388176041335 100.16646779603717) (width 0.15) (layer F.Cu) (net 2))
 (segment (start 96.51388176041335 100.16646779603717) (end 96.29974140653992 100.34606304433892) (width 0.15) (layer F.Cu) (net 2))
 (segment (start 96.29974140653992 100.34606304433892) (end 96.05351722042377 100.38934872524422) (width 0.15) (layer F.Cu) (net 2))
 (segment (start 96.05351722042377 100.38934872524422) (end 95.82381835723191 100.30754093841894) (width 0.15) (layer F.Cu) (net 2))
 (segment (start 95.82381835723191 100.30754093841894) (end 94.23805641079548 99.56736592584818) (width 0.15) (layer F.Cu) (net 2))
 (segment (start 94.23805641079548 99.56736592584818) (end 94.00322889681475 99.48214658086508) (width 0.15) (layer F.Cu) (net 2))
 (segment (start 94.00322889681475 99.48214658086508) (end 93.7557132273198 99.48262145417058) (width 0.15) (layer F.Cu) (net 2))
 (segment (start 93.7557132273198 99.48262145417058) (end 93.55292392006028 99.61850193032818) (width 0.15) (layer F.Cu) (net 2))
 (segment (start 93.55292392006028 99.61850193032818) (end 93.54950779892413 99.86719786017366) (width 0.15) (layer F.Cu) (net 2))
 (segment (start 93.54950779892413 99.86719786017366) (end 93.4279929371264 100.0847269029578) (width 0.15) (layer F.Cu) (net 2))
 (segment (start 93.4279929371264 100.0847269029578) (end 93.27064667472078 100.27900030233862) (width 0.15) (layer F.Cu) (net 2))
 (segment (start 93.27064667472078 100.27900030233862) (end 93.18568675279762 100.51164650724691) (width 0.15) (layer F.Cu) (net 2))
 (segment (start 93.18568675279762 100.51164650724691) (end 93.16700231743735 100.75895590173216) (width 0.15) (layer F.Cu) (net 2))
 (segment (start 93.16700231743735 100.75895590173216) (end 93.16559836397397 101.25895393064295) (width 0.15) (layer F.Cu) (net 2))
 (segment (start 93.16559836397397 101.25895393064295) (end 93.09012163079797 101.5031446924613) (width 0.15) (layer F.Cu) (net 2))
 (segment (start 93.09012163079797 101.5031446924613) (end 93.0455935259553 101.75514406419359) (width 0.15) (layer F.Cu) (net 2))
 (segment (start 93.0455935259553 101.75514406419359) (end 93.0134965262582 102.00728290235756) (width 0.15) (layer F.Cu) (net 2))
 (segment (start 93.0134965262582 102.00728290235756) (end 93.01139027550846 102.75742343857885) (width 0.15) (layer F.Cu) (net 2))
 (segment (start 93.01139027550846 102.75742343857885) (end 93.01104230278581 103.00353259569525) (width 0.15) (layer F.Cu) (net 2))
 (segment (start 93.01104230278581 103.00353259569525) (end 93.00300948880097 103.26499391136493) (width 0.15) (layer F.Cu) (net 2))
 (segment (start 93.00300948880097 103.26499391136493) (end 93.0178912579861 103.50936259698778) (width 0.15) (layer F.Cu) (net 2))
 (segment (start 93.0178912579861 103.50936259698778) (end 93.02390225589447 103.7650745178064) (width 0.15) (layer F.Cu) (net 2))
 (segment (start 93.02390225589447 103.7650745178064) (end 93.04136806084449 104.00825191502668) (width 0.15) (layer F.Cu) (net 2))
 (segment (start 93.04136806084449 104.00825191502668) (end 93.12218593013796 104.25487328117002) (width 0.15) (layer F.Cu) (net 2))
 (segment (start 93.12218593013796 104.25487328117002) (end 93.17148375629735 104.50501269097175) (width 0.15) (layer F.Cu) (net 2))
 (segment (start 93.17148375629735 104.50501269097175) (end 93.16797387263887 105.75500776324873) (width 0.15) (layer F.Cu) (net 2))
 (segment (start 93.16797387263887 105.75500776324873) (end 93.16831448445808 106.00500675370067) (width 0.15) (layer F.Cu) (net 2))
 (segment (start 93.16831448445808 106.00500675370067) (end 93.20518995630486 106.25073918853953) (width 0.15) (layer F.Cu) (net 2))
 (segment (start 93.20518995630486 106.25073918853953) (end 93.30372191687466 106.4741850208825) (width 0.15) (layer F.Cu) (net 2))
 (segment (start 93.30372191687466 106.4741850208825) (end 93.46252911879974 106.66593818858303) (width 0.15) (layer F.Cu) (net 2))
 (segment (start 93.46252911879974 106.66593818858303) (end 93.67833962768758 106.70884824408697) (width 0.15) (layer F.Cu) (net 2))
 (segment (start 93.67833962768758 106.70884824408697) (end 93.94996617746817 106.70219867795089) (width 0.15) (layer F.Cu) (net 2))
 (segment (start 93.94996617746817 106.70219867795089) (end 94.17970584757062 106.73004306580106) (width 0.15) (layer F.Cu) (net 2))
 (segment (start 94.17970584757062 106.73004306580106) (end 94.37971133433058 106.73669641667236) (width 0.15) (layer F.Cu) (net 2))
 (segment (start 94.37971133433058 106.73669641667236) (end 94.66654105188591 106.74956886119084) (width 0.15) (layer F.Cu) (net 2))
 (segment (start 94.66654105188591 106.74956886119084) (end 94.89955501111696 106.85680838875965) (width 0.15) (layer F.Cu) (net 2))
 (segment (start 94.89955501111696 106.85680838875965) (end 95.06598573469071 106.91747684109745) (width 0.15) (layer F.Cu) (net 2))
 (segment (start 95.06598573469071 106.91747684109745) (end 95.25572239430082 107.13883627730924) (width 0.15) (layer F.Cu) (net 2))
 (segment (start 95.25572239430082 107.13883627730924) (end 95.49289321881345 107.21789321881346) (width 0.15) (layer F.Cu) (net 2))
 (segment (start 95.49289321881345 107.21789321881346) (end 96.2 107.925) (width 0.15) (layer F.Cu) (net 2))
 (segment (start 99.0625 99.05) (end 98.59238639567468 99.05) (width 0.15) (layer F.Cu) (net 1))
 (segment (start 98.59238639567468 99.05) (end 98.34785393891335 99.09517121865568) (width 0.15) (layer F.Cu) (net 1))
 (segment (start 98.34785393891335 99.09517121865568) (end 98.17703835719684 99.26552477500454) (width 0.15) (layer F.Cu) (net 1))
 (segment (start 98.17703835719684 99.26552477500454) (end 98.03187006723772 99.46900337447784) (width 0.15) (layer F.Cu) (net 1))
 (segment (start 98.03187006723772 99.46900337447784) (end 97.60194305573943 100.08354610267835) (width 0.15) (layer F.Cu) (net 1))
 (segment (start 97.60194305573943 100.08354610267835) (end 97.56045937405315 100.32444054534635) (width 0.15) (layer F.Cu) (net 1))
 (segment (start 97.56045937405315 100.32444054534635) (end 97.28996625852623 100.27327061012356) (width 0.15) (layer F.Cu) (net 1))
 (segment (start 97.28996625852623 100.27327061012356) (end 97.15128047731376 100.41254795389264) (width 0.15) (layer F.Cu) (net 1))
 (segment (start 97.15128047731376 100.41254795389264) (end 97.09225648044516 100.8049059466396) (width 0.15) (layer F.Cu) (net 1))
 (segment (start 97.09225648044516 100.8049059466396) (end 96.94664889384609 101.00714135071875) (width 0.15) (layer F.Cu) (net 1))
 (segment (start 96.94664889384609 101.00714135071875) (end 96.82081581136735 101.22026020272143) (width 0.15) (layer F.Cu) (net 1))
 (segment (start 96.82081581136735 101.22026020272143) (end 96.63277097921757 101.38205173943848) (width 0.15) (layer F.Cu) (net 1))
 (segment (start 96.63277097921757 101.38205173943848) (end 96.41318268306429 101.54771560808395) (width 0.15) (layer F.Cu) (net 1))
 (segment (start 96.41318268306429 101.54771560808395) (end 96.5161399832145 101.59890387101068) (width 0.15) (layer F.Cu) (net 1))
 (segment (start 96.5161399832145 101.59890387101068) (end 96.6541943582823 101.7125526365596) (width 0.15) (layer F.Cu) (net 1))
 (segment (start 96.6541943582823 101.7125526365596) (end 96.40320595503798 101.63548068905219) (width 0.15) (layer F.Cu) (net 1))
 (segment (start 96.40320595503798 101.63548068905219) (end 96.2422712487669 101.71617716446674) (width 0.15) (layer F.Cu) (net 1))
 (segment (start 96.2422712487669 101.71617716446674) (end 96.18750172978162 101.95476627611366) (width 0.15) (layer F.Cu) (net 1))
 (segment (start 96.18750172978162 101.95476627611366) (end 96.1475378948397 102.19323205580882) (width 0.15) (layer F.Cu) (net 1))
 (segment (start 96.1475378948397 102.19323205580882) (end 96.04573542758034 102.68720141668241) (width 0.15) (layer F.Cu) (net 1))
 (segment (start 96.04573542758034 102.68720141668241) (end 96.28736085684824 102.74056289428162) (width 0.15) (layer F.Cu) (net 1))
 (segment (start 96.28736085684824 102.74056289428162) (end 96.63182157478893 102.57294816496045) (width 0.15) (layer F.Cu) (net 1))
 (segment (start 96.63182157478893 102.57294816496045) (end 96.42851337914645 102.72056516121967) (width 0.15) (layer F.Cu) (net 1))
 (segment (start 96.42851337914645 102.72056516121967) (end 96.2 102.825) (width 0.15) (layer F.Cu) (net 1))
 (gr_line (start 85 115) (end 115 115) (width 0.1) (layer Edge.Cuts))
 (gr_line (start 115 115) (end 115 85) (width 0.1) (layer Edge.Cuts))
 (gr_line (start 115 85) (end 85 85) (width 0.1) (layer Edge.Cuts))
 (gr_line (start 85 85) (end 85 115) (width 0.1) (layer Edge.Cuts)))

